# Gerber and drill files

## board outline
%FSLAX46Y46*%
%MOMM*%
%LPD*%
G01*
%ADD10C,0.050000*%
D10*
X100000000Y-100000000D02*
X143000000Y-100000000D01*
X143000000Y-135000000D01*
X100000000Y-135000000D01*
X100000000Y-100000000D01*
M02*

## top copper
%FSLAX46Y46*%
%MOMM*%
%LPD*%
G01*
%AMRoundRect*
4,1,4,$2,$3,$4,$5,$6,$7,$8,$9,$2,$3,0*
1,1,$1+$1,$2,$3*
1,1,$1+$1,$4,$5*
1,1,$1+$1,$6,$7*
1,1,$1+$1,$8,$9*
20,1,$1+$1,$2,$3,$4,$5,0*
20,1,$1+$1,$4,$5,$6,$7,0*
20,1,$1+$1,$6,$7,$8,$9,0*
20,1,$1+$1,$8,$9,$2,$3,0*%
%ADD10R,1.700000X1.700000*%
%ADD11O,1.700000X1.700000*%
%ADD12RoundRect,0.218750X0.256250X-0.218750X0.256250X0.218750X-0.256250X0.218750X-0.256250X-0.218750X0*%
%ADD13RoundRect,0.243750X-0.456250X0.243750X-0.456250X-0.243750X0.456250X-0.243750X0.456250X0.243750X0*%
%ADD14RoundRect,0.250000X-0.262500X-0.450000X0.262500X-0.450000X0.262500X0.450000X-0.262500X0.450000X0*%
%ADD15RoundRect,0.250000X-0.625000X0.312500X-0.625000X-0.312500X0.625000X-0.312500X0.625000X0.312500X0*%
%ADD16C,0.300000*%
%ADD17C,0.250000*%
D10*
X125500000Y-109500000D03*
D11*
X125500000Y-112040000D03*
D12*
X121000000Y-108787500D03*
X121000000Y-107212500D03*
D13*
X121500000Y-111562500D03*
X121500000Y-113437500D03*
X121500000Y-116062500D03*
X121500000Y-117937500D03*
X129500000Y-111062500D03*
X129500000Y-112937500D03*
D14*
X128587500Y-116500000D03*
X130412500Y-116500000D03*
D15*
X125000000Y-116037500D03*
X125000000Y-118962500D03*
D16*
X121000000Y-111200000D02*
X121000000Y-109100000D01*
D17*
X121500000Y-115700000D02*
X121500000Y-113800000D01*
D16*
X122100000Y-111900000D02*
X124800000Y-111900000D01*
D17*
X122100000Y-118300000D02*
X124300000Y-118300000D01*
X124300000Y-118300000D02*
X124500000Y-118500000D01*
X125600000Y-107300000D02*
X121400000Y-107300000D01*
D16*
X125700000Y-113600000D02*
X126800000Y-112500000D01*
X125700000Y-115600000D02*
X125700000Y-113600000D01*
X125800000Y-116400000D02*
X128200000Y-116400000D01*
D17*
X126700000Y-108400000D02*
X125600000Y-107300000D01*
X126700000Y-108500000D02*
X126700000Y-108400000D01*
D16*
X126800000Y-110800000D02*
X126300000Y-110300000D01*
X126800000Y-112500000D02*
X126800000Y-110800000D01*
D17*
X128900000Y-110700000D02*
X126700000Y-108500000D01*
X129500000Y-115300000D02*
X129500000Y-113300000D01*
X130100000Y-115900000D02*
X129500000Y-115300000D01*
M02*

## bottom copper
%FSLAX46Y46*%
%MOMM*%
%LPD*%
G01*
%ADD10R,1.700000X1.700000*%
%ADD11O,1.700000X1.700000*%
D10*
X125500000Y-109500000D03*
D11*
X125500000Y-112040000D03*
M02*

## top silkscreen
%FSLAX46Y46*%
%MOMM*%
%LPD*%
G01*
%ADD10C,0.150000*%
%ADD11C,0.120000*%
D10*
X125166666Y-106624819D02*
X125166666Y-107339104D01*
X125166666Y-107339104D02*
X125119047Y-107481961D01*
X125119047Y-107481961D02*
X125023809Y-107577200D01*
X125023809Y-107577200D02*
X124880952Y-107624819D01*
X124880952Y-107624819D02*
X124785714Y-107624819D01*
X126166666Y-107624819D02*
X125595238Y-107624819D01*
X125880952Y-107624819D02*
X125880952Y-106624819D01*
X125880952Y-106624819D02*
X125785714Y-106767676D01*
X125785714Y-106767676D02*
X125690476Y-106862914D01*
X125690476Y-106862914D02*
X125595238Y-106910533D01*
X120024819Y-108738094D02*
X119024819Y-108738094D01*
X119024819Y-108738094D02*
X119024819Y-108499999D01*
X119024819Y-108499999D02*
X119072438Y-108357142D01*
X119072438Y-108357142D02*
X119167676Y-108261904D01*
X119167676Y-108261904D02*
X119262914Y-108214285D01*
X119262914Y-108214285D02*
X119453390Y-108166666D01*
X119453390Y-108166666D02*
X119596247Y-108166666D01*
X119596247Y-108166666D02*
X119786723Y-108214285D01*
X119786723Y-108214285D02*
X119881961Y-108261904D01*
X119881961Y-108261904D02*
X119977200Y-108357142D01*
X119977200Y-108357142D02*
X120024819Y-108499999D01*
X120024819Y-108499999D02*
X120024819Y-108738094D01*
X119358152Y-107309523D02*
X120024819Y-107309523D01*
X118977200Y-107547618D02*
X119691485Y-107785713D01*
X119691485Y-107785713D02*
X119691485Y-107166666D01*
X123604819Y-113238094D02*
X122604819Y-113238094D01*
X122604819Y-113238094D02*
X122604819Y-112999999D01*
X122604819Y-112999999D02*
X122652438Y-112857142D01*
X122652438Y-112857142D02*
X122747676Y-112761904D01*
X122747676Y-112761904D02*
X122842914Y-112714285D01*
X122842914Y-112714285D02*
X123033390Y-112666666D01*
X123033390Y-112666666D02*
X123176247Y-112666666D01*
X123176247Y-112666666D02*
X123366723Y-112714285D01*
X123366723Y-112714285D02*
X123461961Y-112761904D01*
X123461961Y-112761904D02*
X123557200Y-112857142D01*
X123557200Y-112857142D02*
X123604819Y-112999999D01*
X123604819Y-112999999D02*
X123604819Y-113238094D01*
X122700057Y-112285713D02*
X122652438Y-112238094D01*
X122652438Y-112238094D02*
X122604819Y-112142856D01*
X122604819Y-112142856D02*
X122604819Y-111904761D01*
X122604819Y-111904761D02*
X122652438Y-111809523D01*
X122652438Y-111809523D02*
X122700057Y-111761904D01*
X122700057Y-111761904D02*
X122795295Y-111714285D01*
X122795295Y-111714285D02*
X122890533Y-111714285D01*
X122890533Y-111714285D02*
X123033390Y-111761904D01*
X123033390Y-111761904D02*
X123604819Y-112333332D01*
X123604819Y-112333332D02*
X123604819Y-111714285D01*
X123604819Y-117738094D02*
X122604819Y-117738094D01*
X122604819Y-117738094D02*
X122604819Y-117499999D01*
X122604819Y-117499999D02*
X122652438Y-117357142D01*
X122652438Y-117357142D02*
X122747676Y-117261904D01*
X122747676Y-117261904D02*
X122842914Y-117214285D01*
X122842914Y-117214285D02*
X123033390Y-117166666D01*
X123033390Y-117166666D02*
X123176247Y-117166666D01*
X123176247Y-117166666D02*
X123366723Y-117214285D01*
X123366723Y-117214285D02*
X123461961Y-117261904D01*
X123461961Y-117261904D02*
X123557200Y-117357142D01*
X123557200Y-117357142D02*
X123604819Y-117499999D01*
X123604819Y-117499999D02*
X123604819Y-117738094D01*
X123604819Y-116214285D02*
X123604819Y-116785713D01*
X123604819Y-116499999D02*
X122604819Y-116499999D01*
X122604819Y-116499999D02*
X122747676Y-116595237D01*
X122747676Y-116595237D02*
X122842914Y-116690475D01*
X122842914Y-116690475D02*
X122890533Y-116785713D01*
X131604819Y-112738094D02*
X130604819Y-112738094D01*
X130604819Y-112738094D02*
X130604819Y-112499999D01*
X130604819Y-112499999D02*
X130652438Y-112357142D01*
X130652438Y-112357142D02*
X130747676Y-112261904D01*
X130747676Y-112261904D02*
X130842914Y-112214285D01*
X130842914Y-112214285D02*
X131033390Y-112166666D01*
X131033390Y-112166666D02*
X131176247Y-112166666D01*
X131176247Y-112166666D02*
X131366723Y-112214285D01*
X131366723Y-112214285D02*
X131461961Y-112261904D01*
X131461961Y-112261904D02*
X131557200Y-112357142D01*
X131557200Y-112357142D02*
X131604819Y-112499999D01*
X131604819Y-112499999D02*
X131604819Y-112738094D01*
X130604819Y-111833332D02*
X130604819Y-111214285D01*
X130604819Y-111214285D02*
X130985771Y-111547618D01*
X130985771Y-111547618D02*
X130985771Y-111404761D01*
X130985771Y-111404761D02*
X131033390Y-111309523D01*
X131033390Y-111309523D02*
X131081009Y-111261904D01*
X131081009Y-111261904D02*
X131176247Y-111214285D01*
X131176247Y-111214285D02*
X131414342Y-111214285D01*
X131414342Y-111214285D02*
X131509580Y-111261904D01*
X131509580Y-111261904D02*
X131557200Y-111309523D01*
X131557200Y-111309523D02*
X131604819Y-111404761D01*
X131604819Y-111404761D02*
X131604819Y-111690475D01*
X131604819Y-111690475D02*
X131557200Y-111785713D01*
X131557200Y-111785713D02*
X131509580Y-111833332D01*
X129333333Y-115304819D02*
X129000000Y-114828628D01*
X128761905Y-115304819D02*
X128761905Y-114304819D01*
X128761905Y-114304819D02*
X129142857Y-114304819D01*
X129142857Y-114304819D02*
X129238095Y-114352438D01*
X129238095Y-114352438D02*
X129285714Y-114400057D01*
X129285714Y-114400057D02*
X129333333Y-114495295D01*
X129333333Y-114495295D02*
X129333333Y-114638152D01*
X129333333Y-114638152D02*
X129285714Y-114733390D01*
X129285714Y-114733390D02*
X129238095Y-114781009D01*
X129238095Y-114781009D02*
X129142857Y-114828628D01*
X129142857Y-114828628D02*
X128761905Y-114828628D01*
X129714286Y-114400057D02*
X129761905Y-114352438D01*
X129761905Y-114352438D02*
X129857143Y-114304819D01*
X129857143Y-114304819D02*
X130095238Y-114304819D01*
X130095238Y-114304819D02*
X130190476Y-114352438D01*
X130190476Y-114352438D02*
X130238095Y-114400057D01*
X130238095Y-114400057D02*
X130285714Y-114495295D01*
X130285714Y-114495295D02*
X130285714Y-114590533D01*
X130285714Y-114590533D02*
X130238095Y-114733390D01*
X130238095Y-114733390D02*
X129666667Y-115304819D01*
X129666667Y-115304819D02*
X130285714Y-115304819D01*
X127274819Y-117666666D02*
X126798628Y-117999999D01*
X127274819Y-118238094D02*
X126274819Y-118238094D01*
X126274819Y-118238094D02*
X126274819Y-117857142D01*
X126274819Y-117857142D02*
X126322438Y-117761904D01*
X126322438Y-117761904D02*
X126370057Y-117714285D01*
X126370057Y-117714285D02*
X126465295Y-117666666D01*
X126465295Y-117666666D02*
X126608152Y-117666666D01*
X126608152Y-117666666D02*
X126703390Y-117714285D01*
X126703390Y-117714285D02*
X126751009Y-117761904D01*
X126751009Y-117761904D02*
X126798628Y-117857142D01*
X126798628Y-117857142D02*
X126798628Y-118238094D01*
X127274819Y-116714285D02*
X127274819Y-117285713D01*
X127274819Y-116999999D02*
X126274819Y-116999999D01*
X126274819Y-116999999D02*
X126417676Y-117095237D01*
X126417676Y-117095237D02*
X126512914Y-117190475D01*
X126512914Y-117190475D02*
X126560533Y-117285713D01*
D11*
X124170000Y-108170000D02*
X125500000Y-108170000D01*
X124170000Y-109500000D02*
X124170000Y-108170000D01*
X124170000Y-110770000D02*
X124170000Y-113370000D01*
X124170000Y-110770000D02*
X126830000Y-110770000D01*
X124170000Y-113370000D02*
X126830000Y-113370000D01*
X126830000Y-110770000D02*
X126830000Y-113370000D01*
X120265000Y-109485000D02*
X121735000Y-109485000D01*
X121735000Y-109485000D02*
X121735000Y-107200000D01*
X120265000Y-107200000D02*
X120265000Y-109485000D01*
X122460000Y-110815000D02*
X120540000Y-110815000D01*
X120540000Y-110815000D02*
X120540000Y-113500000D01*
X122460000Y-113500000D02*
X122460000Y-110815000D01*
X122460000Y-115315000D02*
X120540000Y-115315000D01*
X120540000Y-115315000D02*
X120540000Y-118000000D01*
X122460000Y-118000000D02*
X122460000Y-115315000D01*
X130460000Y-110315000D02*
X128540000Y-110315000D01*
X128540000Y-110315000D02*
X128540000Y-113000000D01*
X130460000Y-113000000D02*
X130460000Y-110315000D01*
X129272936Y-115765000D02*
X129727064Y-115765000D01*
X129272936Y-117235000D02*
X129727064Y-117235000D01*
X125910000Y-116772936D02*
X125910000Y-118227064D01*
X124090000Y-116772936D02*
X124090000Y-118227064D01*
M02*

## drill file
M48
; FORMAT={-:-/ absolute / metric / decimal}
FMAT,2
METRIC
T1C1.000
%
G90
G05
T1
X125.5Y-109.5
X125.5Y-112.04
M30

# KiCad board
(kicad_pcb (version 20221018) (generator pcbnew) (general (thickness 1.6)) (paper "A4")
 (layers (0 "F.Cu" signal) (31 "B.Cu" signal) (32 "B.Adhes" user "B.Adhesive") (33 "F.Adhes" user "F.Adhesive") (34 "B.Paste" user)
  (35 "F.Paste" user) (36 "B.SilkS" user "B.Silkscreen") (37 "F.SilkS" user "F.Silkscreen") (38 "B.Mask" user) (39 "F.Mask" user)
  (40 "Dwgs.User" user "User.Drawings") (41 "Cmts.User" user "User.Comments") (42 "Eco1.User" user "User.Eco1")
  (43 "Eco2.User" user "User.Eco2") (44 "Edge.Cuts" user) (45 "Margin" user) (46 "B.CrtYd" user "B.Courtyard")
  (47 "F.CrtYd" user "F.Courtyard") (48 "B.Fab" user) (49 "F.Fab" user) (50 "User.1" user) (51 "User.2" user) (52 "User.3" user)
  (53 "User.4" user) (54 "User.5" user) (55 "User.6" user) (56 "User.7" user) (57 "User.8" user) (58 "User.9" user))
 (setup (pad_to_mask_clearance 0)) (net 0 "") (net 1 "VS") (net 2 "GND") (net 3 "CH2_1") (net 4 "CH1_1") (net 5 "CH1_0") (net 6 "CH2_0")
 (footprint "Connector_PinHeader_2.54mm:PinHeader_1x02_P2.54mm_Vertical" (layer "F.Cu") (at 125.5 109.5)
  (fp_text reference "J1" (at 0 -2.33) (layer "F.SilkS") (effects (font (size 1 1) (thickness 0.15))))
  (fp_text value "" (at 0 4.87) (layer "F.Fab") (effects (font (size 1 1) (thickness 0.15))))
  (fp_line (start -1.33 -1.33) (end 0 -1.33) (stroke (width 0.12) (type solid)) (layer "F.SilkS"))
  (fp_line (start -1.33 0) (end -1.33 -1.33) (stroke (width 0.12) (type solid)) (layer "F.SilkS"))
  (fp_line (start -1.33 1.27) (end -1.33 3.87) (stroke (width 0.12) (type solid)) (layer "F.SilkS"))
  (fp_line (start -1.33 1.27) (end 1.33 1.27) (stroke (width 0.12) (type solid)) (layer "F.SilkS"))
  (fp_line (start -1.33 3.87) (end 1.33 3.87) (stroke (width 0.12) (type solid)) (layer "F.SilkS"))
  (fp_line (start 1.33 1.27) (end 1.33 3.87) (stroke (width 0.12) (type solid)) (layer "F.SilkS"))
  (pad "1" thru_hole rect (at 0 0) (size 1.7 1.7) (drill 1) (layers "*.Cu" "*.Mask") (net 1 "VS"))
  (pad "2" thru_hole oval (at 0 2.54) (size 1.7 1.7) (drill 1) (layers "*.Cu" "*.Mask") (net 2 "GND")))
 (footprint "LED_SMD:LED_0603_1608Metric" (layer "F.Cu") (at 121 108 90)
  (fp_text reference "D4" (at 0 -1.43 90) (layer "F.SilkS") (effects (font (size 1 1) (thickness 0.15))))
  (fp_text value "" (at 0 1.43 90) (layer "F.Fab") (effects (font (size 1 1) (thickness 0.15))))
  (fp_line (start -1.485 -0.735) (end -1.485 0.735) (stroke (width 0.12) (type solid)) (layer "F.SilkS"))
  (fp_line (start -1.485 0.735) (end 0.8 0.735) (stroke (width 0.12) (type solid)) (layer "F.SilkS"))
  (fp_line (start 0.8 -0.735) (end -1.485 -0.735) (stroke (width 0.12) (type solid)) (layer "F.SilkS"))
  (pad "1" smd roundrect (at -0.7875 0 90) (size 0.875 0.95) (layers "F.Cu" "F.Paste" "F.Mask") (roundrect_rratio 0.25) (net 2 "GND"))
  (pad "2" smd roundrect (at 0.7875 0 90) (size 0.875 0.95) (layers "F.Cu" "F.Paste" "F.Mask") (roundrect_rratio 0.25) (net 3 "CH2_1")))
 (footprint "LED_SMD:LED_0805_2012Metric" (layer "F.Cu") (at 121.5 112.5 -90)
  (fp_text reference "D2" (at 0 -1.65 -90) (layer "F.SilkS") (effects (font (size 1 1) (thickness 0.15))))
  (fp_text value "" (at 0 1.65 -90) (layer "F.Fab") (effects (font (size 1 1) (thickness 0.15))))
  (fp_line (start -1.685 -0.96) (end -1.685 0.96) (stroke (width 0.12) (type solid)) (layer "F.SilkS"))
  (fp_line (start -1.685 0.96) (end 1 0.96) (stroke (width 0.12) (type solid)) (layer "F.SilkS"))
  (fp_line (start 1 -0.96) (end -1.685 -0.96) (stroke (width 0.12) (type solid)) (layer "F.SilkS"))
  (pad "1" smd roundrect (at -0.9375 0 270) (size 0.975 1.4) (layers "F.Cu" "F.Paste" "F.Mask") (roundrect_rratio 0.25) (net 2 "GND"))
  (pad "2" smd roundrect (at 0.9375 0 270) (size 0.975 1.4) (layers "F.Cu" "F.Paste" "F.Mask") (roundrect_rratio 0.25) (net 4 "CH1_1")))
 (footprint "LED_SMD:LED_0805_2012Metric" (layer "F.Cu") (at 121.5 117 -90)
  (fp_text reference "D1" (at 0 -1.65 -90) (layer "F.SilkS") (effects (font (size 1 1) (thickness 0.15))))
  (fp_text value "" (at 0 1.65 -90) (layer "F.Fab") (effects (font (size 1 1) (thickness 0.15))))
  (fp_line (start -1.685 -0.96) (end -1.685 0.96) (stroke (width 0.12) (type solid)) (layer "F.SilkS"))
  (fp_line (start -1.685 0.96) (end 1 0.96) (stroke (width 0.12) (type solid)) (layer "F.SilkS"))
  (fp_line (start 1 -0.96) (end -1.685 -0.96) (stroke (width 0.12) (type solid)) (layer "F.SilkS"))
  (pad "1" smd roundrect (at -0.9375 0 270) (size 0.975 1.4) (layers "F.Cu" "F.Paste" "F.Mask") (roundrect_rratio 0.25) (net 4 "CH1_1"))
  (pad "2" smd roundrect (at 0.9375 0 270) (size 0.975 1.4) (layers "F.Cu" "F.Paste" "F.Mask") (roundrect_rratio 0.25) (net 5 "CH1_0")))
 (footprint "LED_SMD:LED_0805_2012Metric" (layer "F.Cu") (at 129.5 112 -90)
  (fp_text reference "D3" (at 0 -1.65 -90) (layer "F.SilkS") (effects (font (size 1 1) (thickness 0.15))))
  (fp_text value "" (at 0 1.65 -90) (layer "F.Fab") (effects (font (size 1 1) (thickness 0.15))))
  (fp_line (start -1.685 -0.96) (end -1.685 0.96) (stroke (width 0.12) (type solid)) (layer "F.SilkS"))
  (fp_line (start -1.685 0.96) (end 1 0.96) (stroke (width 0.12) (type solid)) (layer "F.SilkS"))
  (fp_line (start 1 -0.96) (end -1.685 -0.96) (stroke (width 0.12) (type solid)) (layer "F.SilkS"))
  (pad "1" smd roundrect (at -0.9375 0 270) (size 0.975 1.4) (layers "F.Cu" "F.Paste" "F.Mask") (roundrect_rratio 0.25) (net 3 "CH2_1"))
  (pad "2" smd roundrect (at 0.9375 0 270) (size 0.975 1.4) (layers "F.Cu" "F.Paste" "F.Mask") (roundrect_rratio 0.25) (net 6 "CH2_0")))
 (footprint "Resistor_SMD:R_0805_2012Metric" (layer "F.Cu") (at 129.5 116.5)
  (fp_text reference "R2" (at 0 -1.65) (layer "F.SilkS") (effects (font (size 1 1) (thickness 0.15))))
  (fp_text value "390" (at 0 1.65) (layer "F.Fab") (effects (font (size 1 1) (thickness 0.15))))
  (fp_line (start -0.227064 -0.735) (end 0.227064 -0.735) (stroke (width 0.12) (type solid)) (layer "F.SilkS"))
  (fp_line (start -0.227064 0.735) (end 0.227064 0.735) (stroke (width 0.12) (type solid)) (layer "F.SilkS"))
  (pad "1" smd roundrect (at -0.9125 0) (size 1.025 1.4) (layers "F.Cu" "F.Paste" "F.Mask") (roundrect_rratio 0.243902) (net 1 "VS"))
  (pad "2" smd roundrect (at 0.9125 0) (size 1.025 1.4) (layers "F.Cu" "F.Paste" "F.Mask") (roundrect_rratio 0.243902) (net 6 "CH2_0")))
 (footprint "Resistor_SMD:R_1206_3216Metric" (layer "F.Cu") (at 125 117.5 -90)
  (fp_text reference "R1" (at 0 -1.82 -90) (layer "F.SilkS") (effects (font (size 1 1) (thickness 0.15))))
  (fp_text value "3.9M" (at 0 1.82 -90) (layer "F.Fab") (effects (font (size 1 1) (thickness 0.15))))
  (fp_line (start -0.727064 -0.91) (end 0.727064 -0.91) (stroke (width 0.12) (type solid)) (layer "F.SilkS"))
  (fp_line (start -0.727064 0.91) (end 0.727064 0.91) (stroke (width 0.12) (type solid)) (layer "F.SilkS"))
  (pad "1" smd roundrect (at -1.4625 0 270) (size 1.125 1.75) (layers "F.Cu" "F.Paste" "F.Mask") (roundrect_rratio 0.222222) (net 1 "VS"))
  (pad "2" smd roundrect (at 1.4625 0 270) (size 1.125 1.75) (layers "F.Cu" "F.Paste" "F.Mask") (roundrect_rratio 0.222222) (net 5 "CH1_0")))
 (gr_rect (start 100 100) (end 143 135) (stroke (width 0.05) (type default)) (fill none) (layer "Edge.Cuts"))
 (segment (start 121 111.2) (end 121 109.1) (width 0.3) (layer "F.Cu") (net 2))
 (segment (start 121.5 115.7) (end 121.5 113.8) (width 0.25) (layer "F.Cu") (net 4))
 (segment (start 122.1 111.9) (end 124.8 111.9) (width 0.3) (layer "F.Cu") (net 2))
 (segment (start 122.1 118.3) (end 124.3 118.3) (width 0.25) (layer "F.Cu") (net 5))
 (segment (start 124.3 118.3) (end 124.5 118.5) (width 0.25) (layer "F.Cu") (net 5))
 (segment (start 125.6 107.3) (end 121.4 107.3) (width 0.25) (layer "F.Cu") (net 3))
 (segment (start 125.7 113.6) (end 126.8 112.5) (width 0.3) (layer "F.Cu") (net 1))
 (segment (start 125.7 115.6) (end 125.7 113.6) (width 0.3) (layer "F.Cu") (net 1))
 (segment (start 125.8 116.4) (end 128.2 116.4) (width 0.3) (layer "F.Cu") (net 1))
 (segment (start 126.7 108.4) (end 125.6 107.3) (width 0.25) (layer "F.Cu") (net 3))
 (segment (start 126.7 108.5) (end 126.7 108.4) (width 0.25) (layer "F.Cu") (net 3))
 (segment (start 126.8 110.8) (end 126.3 110.3) (width 0.3) (layer "F.Cu") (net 1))
 (segment (start 126.8 112.5) (end 126.8 110.8) (width 0.3) (layer "F.Cu") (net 1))
 (segment (start 128.9 110.7) (end 126.7 108.5) (width 0.25) (layer "F.Cu") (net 3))
 (segment (start 129.5 115.3) (end 129.5 113.3) (width 0.25) (layer "F.Cu") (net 6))
 (segment (start 130.1 115.9) (end 129.5 115.3) (width 0.25) (layer "F.Cu") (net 6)))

